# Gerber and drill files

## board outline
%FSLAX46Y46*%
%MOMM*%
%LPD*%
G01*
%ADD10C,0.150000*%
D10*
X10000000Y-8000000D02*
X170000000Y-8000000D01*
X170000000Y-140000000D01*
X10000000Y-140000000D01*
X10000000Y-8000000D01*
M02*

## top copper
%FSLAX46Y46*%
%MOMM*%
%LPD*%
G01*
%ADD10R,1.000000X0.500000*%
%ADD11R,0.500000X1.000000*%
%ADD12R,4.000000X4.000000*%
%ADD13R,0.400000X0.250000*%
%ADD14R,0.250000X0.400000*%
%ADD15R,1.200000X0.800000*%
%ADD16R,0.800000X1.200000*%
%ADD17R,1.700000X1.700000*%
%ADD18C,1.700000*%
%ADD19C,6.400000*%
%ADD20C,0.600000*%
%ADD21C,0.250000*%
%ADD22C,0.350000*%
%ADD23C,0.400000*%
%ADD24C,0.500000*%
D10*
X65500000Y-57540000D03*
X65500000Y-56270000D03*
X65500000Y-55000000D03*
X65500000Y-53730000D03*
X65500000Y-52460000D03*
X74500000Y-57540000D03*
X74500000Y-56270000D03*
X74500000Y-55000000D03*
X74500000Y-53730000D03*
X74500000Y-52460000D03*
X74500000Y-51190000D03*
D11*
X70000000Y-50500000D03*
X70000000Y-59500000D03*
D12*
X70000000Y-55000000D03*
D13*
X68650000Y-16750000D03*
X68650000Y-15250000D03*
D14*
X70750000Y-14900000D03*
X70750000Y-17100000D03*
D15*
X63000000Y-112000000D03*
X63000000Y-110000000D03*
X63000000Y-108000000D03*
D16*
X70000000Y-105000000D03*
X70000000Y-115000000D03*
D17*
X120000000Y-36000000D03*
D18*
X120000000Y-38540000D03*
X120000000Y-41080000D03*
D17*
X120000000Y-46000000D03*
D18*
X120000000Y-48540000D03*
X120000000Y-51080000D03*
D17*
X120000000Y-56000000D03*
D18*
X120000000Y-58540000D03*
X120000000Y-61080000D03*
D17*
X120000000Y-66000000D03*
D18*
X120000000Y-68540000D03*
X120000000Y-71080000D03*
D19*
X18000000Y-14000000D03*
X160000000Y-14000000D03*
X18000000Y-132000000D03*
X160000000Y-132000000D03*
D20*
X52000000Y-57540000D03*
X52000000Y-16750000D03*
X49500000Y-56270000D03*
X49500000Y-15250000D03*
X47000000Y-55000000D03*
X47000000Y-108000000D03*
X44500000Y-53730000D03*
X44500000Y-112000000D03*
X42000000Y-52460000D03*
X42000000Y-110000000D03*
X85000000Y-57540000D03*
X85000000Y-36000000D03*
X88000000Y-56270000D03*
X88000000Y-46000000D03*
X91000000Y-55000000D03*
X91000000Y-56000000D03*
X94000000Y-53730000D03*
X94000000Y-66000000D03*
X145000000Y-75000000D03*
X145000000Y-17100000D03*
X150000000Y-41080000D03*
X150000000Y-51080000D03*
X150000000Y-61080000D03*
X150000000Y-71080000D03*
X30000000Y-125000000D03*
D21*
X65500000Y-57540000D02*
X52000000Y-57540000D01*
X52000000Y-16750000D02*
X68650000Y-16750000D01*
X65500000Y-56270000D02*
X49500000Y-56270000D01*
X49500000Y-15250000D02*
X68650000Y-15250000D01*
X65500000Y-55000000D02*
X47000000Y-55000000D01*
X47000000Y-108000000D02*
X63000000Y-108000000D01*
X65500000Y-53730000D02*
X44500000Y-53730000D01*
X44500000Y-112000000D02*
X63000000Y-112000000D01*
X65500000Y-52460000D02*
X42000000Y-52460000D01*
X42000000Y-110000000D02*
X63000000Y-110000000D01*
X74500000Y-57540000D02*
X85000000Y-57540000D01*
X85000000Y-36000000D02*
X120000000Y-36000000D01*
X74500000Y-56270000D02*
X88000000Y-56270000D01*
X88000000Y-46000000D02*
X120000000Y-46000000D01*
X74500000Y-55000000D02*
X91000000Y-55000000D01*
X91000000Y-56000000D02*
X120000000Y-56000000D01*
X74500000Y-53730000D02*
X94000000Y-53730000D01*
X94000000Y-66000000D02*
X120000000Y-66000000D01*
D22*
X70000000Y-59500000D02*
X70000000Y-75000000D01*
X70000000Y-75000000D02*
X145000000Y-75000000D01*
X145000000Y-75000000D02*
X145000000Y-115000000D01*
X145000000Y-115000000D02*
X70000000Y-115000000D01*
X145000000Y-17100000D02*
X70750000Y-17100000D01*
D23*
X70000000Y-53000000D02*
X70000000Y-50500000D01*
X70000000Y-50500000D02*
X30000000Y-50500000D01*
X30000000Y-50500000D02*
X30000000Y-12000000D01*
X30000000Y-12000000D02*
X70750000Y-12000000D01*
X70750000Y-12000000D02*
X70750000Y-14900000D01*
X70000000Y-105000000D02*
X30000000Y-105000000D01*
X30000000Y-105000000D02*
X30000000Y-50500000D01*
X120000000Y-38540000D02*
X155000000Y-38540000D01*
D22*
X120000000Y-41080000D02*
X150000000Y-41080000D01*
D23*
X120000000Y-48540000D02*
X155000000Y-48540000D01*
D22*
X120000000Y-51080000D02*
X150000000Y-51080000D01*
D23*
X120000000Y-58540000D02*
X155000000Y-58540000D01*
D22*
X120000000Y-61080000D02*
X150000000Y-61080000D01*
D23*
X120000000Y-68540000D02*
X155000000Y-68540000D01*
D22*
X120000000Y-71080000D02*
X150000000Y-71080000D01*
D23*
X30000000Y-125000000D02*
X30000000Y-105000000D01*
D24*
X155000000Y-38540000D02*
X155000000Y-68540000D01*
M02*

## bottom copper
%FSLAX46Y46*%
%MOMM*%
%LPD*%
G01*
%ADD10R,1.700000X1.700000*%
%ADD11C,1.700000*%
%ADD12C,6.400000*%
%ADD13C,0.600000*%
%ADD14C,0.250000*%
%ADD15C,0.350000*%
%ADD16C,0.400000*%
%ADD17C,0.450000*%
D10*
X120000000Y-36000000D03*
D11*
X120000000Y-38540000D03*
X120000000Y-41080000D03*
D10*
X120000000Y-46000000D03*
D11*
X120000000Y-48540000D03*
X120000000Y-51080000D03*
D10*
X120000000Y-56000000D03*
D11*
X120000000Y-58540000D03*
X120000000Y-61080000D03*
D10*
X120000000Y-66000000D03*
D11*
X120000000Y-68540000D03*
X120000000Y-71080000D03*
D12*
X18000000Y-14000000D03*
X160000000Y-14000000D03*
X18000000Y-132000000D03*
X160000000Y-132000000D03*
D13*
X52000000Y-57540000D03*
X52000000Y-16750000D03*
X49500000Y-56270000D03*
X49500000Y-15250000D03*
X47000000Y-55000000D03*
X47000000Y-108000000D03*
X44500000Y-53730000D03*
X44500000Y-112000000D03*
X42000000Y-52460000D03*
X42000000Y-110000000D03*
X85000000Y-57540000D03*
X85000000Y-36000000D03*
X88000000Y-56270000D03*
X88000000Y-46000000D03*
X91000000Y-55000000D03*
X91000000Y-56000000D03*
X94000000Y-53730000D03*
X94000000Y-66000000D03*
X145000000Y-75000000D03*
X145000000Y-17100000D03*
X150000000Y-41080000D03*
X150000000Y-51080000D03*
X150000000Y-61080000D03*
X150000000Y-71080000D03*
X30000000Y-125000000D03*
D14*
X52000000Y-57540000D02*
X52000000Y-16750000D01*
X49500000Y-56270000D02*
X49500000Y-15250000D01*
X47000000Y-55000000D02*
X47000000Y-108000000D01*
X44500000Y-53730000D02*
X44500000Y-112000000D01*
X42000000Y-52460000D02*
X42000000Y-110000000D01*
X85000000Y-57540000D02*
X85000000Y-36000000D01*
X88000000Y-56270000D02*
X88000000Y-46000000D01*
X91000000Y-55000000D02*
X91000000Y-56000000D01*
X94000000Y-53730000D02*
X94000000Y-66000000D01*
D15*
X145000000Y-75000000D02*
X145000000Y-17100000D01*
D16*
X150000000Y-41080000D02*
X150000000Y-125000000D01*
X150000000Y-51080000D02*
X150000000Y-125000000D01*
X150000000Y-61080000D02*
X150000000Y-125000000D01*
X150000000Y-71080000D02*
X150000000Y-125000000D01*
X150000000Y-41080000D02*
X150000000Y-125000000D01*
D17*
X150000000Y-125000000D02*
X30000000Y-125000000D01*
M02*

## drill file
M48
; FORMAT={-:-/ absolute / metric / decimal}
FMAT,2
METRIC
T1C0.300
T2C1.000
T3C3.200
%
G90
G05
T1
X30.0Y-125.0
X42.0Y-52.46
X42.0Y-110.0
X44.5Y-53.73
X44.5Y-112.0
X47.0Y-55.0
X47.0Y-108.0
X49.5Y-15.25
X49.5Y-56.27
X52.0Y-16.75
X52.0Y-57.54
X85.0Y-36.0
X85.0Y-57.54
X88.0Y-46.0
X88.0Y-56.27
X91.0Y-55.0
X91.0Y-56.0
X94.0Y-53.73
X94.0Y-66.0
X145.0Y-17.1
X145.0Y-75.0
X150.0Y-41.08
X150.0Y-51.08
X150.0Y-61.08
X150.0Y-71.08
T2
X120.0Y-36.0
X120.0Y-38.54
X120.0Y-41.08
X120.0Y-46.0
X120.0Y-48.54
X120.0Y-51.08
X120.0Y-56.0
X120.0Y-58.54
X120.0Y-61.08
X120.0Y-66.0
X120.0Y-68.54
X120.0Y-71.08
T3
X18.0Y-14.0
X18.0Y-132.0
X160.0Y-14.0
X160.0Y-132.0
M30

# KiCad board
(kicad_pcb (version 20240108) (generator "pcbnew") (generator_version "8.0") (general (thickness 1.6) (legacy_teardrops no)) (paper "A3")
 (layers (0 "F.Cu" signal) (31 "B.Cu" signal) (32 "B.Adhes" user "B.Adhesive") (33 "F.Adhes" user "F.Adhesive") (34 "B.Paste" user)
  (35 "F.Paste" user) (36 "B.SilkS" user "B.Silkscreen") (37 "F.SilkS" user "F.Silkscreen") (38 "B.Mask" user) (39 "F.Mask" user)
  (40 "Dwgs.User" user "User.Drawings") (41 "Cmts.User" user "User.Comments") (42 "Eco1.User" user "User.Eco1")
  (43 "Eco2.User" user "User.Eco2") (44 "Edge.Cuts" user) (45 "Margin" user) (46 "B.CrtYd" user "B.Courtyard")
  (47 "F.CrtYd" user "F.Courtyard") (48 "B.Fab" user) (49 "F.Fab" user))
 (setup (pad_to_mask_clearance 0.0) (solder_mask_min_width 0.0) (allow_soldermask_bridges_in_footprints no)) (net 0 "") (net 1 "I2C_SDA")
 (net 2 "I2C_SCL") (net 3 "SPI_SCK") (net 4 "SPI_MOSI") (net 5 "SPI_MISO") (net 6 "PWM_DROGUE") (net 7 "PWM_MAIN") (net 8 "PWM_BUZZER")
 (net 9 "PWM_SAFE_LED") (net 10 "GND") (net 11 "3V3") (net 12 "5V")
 (gr_rect (start 10 8) (end 170 140) (stroke (width 0.15) (type solid)) (fill none) (layer "Edge.Cuts"))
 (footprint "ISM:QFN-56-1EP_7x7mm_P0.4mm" (layer "F.Cu") (at 70 55)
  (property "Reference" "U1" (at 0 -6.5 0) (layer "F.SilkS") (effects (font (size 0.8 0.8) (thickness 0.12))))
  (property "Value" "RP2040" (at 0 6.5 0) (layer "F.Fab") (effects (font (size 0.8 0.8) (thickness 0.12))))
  (pad "1" smd rect (at -4.5 2.54) (size 1.0 0.5) (layers "F.Cu" "F.Paste" "F.Mask") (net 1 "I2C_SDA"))
  (pad "2" smd rect (at -4.5 1.27) (size 1.0 0.5) (layers "F.Cu" "F.Paste" "F.Mask") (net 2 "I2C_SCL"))
  (pad "3" smd rect (at -4.5 0) (size 1.0 0.5) (layers "F.Cu" "F.Paste" "F.Mask") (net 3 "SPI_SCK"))
  (pad "4" smd rect (at -4.5 -1.27) (size 1.0 0.5) (layers "F.Cu" "F.Paste" "F.Mask") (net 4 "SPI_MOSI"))
  (pad "5" smd rect (at -4.5 -2.54) (size 1.0 0.5) (layers "F.Cu" "F.Paste" "F.Mask") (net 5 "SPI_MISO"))
  (pad "6" smd rect (at 4.5 2.54) (size 1.0 0.5) (layers "F.Cu" "F.Paste" "F.Mask") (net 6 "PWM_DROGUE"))
  (pad "7" smd rect (at 4.5 1.27) (size 1.0 0.5) (layers "F.Cu" "F.Paste" "F.Mask") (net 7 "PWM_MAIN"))
  (pad "8" smd rect (at 4.5 0) (size 1.0 0.5) (layers "F.Cu" "F.Paste" "F.Mask") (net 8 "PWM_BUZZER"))
  (pad "9" smd rect (at 4.5 -1.27) (size 1.0 0.5) (layers "F.Cu" "F.Paste" "F.Mask") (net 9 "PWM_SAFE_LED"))
  (pad "12" smd rect (at 4.5 -2.54) (size 1.0 0.5) (layers "F.Cu" "F.Paste" "F.Mask"))
  (pad "13" smd rect (at 4.5 -3.81) (size 1.0 0.5) (layers "F.Cu" "F.Paste" "F.Mask"))
  (pad "10" smd rect (at 0 -4.5) (size 0.5 1.0) (layers "F.Cu" "F.Paste" "F.Mask") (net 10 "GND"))
  (pad "11" smd rect (at 0 4.5) (size 0.5 1.0) (layers "F.Cu" "F.Paste" "F.Mask") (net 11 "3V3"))
  (pad "EP" smd rect (at 0 0) (size 4 4) (layers "F.Cu" "F.Paste" "F.Mask") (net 10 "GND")))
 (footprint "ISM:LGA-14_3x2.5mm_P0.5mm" (layer "F.Cu") (at 70 16)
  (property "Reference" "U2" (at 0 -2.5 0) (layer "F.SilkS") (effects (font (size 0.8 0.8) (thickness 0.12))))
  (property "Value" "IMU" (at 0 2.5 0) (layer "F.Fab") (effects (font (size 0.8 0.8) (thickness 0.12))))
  (pad "1" smd rect (at -1.35 0.75) (size 0.4 0.25) (layers "F.Cu" "F.Paste" "F.Mask") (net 1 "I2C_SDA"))
  (pad "2" smd rect (at -1.35 -0.75) (size 0.4 0.25) (layers "F.Cu" "F.Paste" "F.Mask") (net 2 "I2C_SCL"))
  (pad "3" smd rect (at 0.75 -1.1) (size 0.25 0.4) (layers "F.Cu" "F.Paste" "F.Mask") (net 10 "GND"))
  (pad "4" smd rect (at 0.75 1.1) (size 0.25 0.4) (layers "F.Cu" "F.Paste" "F.Mask") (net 11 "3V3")))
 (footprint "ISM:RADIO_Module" (layer "F.Cu") (at 70 110)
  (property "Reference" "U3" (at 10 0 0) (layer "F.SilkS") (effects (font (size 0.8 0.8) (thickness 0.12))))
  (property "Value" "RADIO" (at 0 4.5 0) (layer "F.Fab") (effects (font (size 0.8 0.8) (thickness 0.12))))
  (pad "1" smd rect (at -7 2) (size 1.2 0.8) (layers "F.Cu" "F.Paste" "F.Mask") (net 4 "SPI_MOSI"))
  (pad "2" smd rect (at -7 0) (size 1.2 0.8) (layers "F.Cu" "F.Paste" "F.Mask") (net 5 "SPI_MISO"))
  (pad "3" smd rect (at -7 -2) (size 1.2 0.8) (layers "F.Cu" "F.Paste" "F.Mask") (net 3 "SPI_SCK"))
  (pad "4" smd rect (at 0 -5) (size 0.8 1.2) (layers "F.Cu" "F.Paste" "F.Mask") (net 10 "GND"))
  (pad "5" smd rect (at 0 5) (size 0.8 1.2) (layers "F.Cu" "F.Paste" "F.Mask") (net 11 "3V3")))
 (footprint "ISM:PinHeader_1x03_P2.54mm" (layer "F.Cu") (at 120 36)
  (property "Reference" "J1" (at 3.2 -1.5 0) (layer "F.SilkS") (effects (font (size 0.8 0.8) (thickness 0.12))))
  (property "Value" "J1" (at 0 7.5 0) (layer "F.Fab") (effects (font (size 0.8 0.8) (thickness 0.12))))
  (pad "1" thru_hole rect (at 0 0) (size 1.7 1.7) (drill 1.0) (layers "*.Cu" "*.Mask") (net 6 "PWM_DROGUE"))
  (pad "2" thru_hole circle (at 0 2.54) (size 1.7 1.7) (drill 1.0) (layers "*.Cu" "*.Mask") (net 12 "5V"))
  (pad "3" thru_hole circle (at 0 5.08) (size 1.7 1.7) (drill 1.0) (layers "*.Cu" "*.Mask") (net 10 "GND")))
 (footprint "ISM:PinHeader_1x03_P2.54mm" (layer "F.Cu") (at 120 46)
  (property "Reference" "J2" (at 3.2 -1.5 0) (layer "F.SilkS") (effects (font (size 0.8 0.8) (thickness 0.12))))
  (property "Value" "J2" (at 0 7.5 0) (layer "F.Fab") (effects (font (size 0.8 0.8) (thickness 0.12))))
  (pad "1" thru_hole rect (at 0 0) (size 1.7 1.7) (drill 1.0) (layers "*.Cu" "*.Mask") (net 7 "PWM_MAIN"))
  (pad "2" thru_hole circle (at 0 2.54) (size 1.7 1.7) (drill 1.0) (layers "*.Cu" "*.Mask") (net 12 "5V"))
  (pad "3" thru_hole circle (at 0 5.08) (size 1.7 1.7) (drill 1.0) (layers "*.Cu" "*.Mask") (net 10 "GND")))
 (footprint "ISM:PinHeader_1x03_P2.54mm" (layer "F.Cu") (at 120 56)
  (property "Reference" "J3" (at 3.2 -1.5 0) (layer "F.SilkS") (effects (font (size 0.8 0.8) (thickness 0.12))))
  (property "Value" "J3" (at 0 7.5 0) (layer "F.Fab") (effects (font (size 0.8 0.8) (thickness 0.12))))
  (pad "1" thru_hole rect (at 0 0) (size 1.7 1.7) (drill 1.0) (layers "*.Cu" "*.Mask") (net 8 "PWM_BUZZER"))
  (pad "2" thru_hole circle (at 0 2.54) (size 1.7 1.7) (drill 1.0) (layers "*.Cu" "*.Mask") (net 12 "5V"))
  (pad "3" thru_hole circle (at 0 5.08) (size 1.7 1.7) (drill 1.0) (layers "*.Cu" "*.Mask") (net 10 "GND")))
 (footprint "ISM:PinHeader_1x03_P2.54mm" (layer "F.Cu") (at 120 66)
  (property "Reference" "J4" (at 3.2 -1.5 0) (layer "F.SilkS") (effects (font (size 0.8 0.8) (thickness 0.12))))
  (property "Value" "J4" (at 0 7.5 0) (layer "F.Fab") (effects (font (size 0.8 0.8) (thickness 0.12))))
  (pad "1" thru_hole rect (at 0 0) (size 1.7 1.7) (drill 1.0) (layers "*.Cu" "*.Mask") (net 9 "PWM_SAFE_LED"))
  (pad "2" thru_hole circle (at 0 2.54) (size 1.7 1.7) (drill 1.0) (layers "*.Cu" "*.Mask") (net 12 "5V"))
  (pad "3" thru_hole circle (at 0 5.08) (size 1.7 1.7) (drill 1.0) (layers "*.Cu" "*.Mask") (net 10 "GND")))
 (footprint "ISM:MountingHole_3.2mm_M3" (layer "F.Cu") (at 18 14)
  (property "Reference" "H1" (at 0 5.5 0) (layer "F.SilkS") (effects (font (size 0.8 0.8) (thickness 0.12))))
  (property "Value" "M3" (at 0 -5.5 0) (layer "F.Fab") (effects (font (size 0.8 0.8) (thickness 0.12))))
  (pad "" thru_hole circle (at 0 0) (size 6.4 6.4) (drill 3.2) (layers "*.Cu" "*.Mask")))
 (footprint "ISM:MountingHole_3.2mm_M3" (layer "F.Cu") (at 160 14)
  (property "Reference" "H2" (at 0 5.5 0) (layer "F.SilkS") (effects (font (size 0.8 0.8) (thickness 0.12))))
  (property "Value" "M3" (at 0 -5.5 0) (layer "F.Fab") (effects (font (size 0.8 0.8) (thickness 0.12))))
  (pad "" thru_hole circle (at 0 0) (size 6.4 6.4) (drill 3.2) (layers "*.Cu" "*.Mask")))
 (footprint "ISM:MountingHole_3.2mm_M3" (layer "F.Cu") (at 18 132)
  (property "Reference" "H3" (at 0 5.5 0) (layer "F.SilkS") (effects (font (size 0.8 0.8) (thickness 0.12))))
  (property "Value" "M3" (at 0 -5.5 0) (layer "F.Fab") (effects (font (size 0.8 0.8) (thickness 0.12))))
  (pad "" thru_hole circle (at 0 0) (size 6.4 6.4) (drill 3.2) (layers "*.Cu" "*.Mask")))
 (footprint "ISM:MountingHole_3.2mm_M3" (layer "F.Cu") (at 160 132)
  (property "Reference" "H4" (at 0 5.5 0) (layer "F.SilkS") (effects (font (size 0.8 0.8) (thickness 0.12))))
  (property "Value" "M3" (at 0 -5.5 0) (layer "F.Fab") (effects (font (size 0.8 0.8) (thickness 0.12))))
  (pad "" thru_hole circle (at 0 0) (size 6.4 6.4) (drill 3.2) (layers "*.Cu" "*.Mask")))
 (segment (start 65.5 57.54) (end 52.0 57.54) (width 0.25) (layer "F.Cu") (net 1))
 (segment (start 52.0 57.54) (end 52.0 16.75) (width 0.25) (layer "B.Cu") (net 1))
 (segment (start 52.0 16.75) (end 68.65 16.75) (width 0.25) (layer "F.Cu") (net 1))
 (segment (start 65.5 56.27) (end 49.5 56.27) (width 0.25) (layer "F.Cu") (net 2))
 (segment (start 49.5 56.27) (end 49.5 15.25) (width 0.25) (layer "B.Cu") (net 2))
 (segment (start 49.5 15.25) (end 68.65 15.25) (width 0.25) (layer "F.Cu") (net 2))
 (segment (start 65.5 55) (end 47.0 55) (width 0.25) (layer "F.Cu") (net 3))
 (segment (start 47.0 55) (end 47.0 108) (width 0.25) (layer "B.Cu") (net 3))
 (segment (start 47.0 108) (end 63 108) (width 0.25) (layer "F.Cu") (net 3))
 (segment (start 65.5 53.73) (end 44.5 53.73) (width 0.25) (layer "F.Cu") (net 4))
 (segment (start 44.5 53.73) (end 44.5 112) (width 0.25) (layer "B.Cu") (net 4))
 (segment (start 44.5 112) (end 63 112) (width 0.25) (layer "F.Cu") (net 4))
 (segment (start 65.5 52.46) (end 42.0 52.46) (width 0.25) (layer "F.Cu") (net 5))
 (segment (start 42.0 52.46) (end 42.0 110) (width 0.25) (layer "B.Cu") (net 5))
 (segment (start 42.0 110) (end 63 110) (width 0.25) (layer "F.Cu") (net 5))
 (segment (start 74.5 57.54) (end 85 57.54) (width 0.25) (layer "F.Cu") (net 6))
 (segment (start 85 57.54) (end 85 36) (width 0.25) (layer "B.Cu") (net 6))
 (segment (start 85 36) (end 120 36) (width 0.25) (layer "F.Cu") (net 6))
 (segment (start 74.5 56.27) (end 88 56.27) (width 0.25) (layer "F.Cu") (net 7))
 (segment (start 88 56.27) (end 88 46) (width 0.25) (layer "B.Cu") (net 7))
 (segment (start 88 46) (end 120 46) (width 0.25) (layer "F.Cu") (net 7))
 (segment (start 74.5 55) (end 91 55) (width 0.25) (layer "F.Cu") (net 8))
 (segment (start 91 55) (end 91 56) (width 0.25) (layer "B.Cu") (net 8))
 (segment (start 91 56) (end 120 56) (width 0.25) (layer "F.Cu") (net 8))
 (segment (start 74.5 53.73) (end 94 53.73) (width 0.25) (layer "F.Cu") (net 9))
 (segment (start 94 53.73) (end 94 66) (width 0.25) (layer "B.Cu") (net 9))
 (segment (start 94 66) (end 120 66) (width 0.25) (layer "F.Cu") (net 9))
 (segment (start 70 59.5) (end 70 75) (width 0.35) (layer "F.Cu") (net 11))
 (segment (start 70 75) (end 145 75) (width 0.35) (layer "F.Cu") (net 11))
 (segment (start 145 75) (end 145 115) (width 0.35) (layer "F.Cu") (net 11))
 (segment (start 145 115) (end 70 115) (width 0.35) (layer "F.Cu") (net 11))
 (segment (start 145 75) (end 145 17.1) (width 0.35) (layer "B.Cu") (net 11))
 (segment (start 145 17.1) (end 70.75 17.1) (width 0.35) (layer "F.Cu") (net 11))
 (segment (start 70 53) (end 70 50.5) (width 0.4) (layer "F.Cu") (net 10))
 (segment (start 70 50.5) (end 30 50.5) (width 0.4) (layer "F.Cu") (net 10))
 (segment (start 30 50.5) (end 30 12) (width 0.4) (layer "F.Cu") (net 10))
 (segment (start 30 12) (end 70.75 12) (width 0.4) (layer "F.Cu") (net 10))
 (segment (start 70.75 12) (end 70.75 14.9) (width 0.4) (layer "F.Cu") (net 10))
 (segment (start 70 105) (end 30 105) (width 0.4) (layer "F.Cu") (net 10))
 (segment (start 30 105) (end 30 50.5) (width 0.4) (layer "F.Cu") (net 10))
 (segment (start 120 38.54) (end 155 38.54) (width 0.4) (layer "F.Cu") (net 12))
 (segment (start 120 41.08) (end 150 41.08) (width 0.35) (layer "F.Cu") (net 10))
 (segment (start 150 41.08) (end 150 125) (width 0.4) (layer "B.Cu") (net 10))
 (segment (start 120 48.54) (end 155 48.54) (width 0.4) (layer "F.Cu") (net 12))
 (segment (start 120 51.08) (end 150 51.08) (width 0.35) (layer "F.Cu") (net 10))
 (segment (start 150 51.08) (end 150 125) (width 0.4) (layer "B.Cu") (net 10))
 (segment (start 120 58.54) (end 155 58.54) (width 0.4) (layer "F.Cu") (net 12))
 (segment (start 120 61.08) (end 150 61.08) (width 0.35) (layer "F.Cu") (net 10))
 (segment (start 150 61.08) (end 150 125) (width 0.4) (layer "B.Cu") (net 10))
 (segment (start 120 68.54) (end 155 68.54) (width 0.4) (layer "F.Cu") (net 12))
 (segment (start 120 71.08) (end 150 71.08) (width 0.35) (layer "F.Cu") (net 10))
 (segment (start 150 71.08) (end 150 125) (width 0.4) (layer "B.Cu") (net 10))
 (segment (start 150 41.08) (end 150 125) (width 0.4) (layer "B.Cu") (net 10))
 (segment (start 150 125) (end 30 125) (width 0.45) (layer "B.Cu") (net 10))
 (segment (start 30 125) (end 30 105) (width 0.4) (layer "F.Cu") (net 10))
 (segment (start 155 38.54) (end 155 68.54) (width 0.5) (layer "F.Cu") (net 12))
 (via (at 52.0 57.54) (size 0.6) (drill 0.3) (layers "F.Cu" "B.Cu") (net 1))
 (via (at 52.0 16.75) (size 0.6) (drill 0.3) (layers "F.Cu" "B.Cu") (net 1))
 (via (at 49.5 56.27) (size 0.6) (drill 0.3) (layers "F.Cu" "B.Cu") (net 2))
 (via (at 49.5 15.25) (size 0.6) (drill 0.3) (layers "F.Cu" "B.Cu") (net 2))
 (via (at 47.0 55) (size 0.6) (drill 0.3) (layers "F.Cu" "B.Cu") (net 3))
 (via (at 47.0 108) (size 0.6) (drill 0.3) (layers "F.Cu" "B.Cu") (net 3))
 (via (at 44.5 53.73) (size 0.6) (drill 0.3) (layers "F.Cu" "B.Cu") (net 4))
 (via (at 44.5 112) (size 0.6) (drill 0.3) (layers "F.Cu" "B.Cu") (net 4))
 (via (at 42.0 52.46) (size 0.6) (drill 0.3) (layers "F.Cu" "B.Cu") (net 5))
 (via (at 42.0 110) (size 0.6) (drill 0.3) (layers "F.Cu" "B.Cu") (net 5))
 (via (at 85 57.54) (size 0.6) (drill 0.3) (layers "F.Cu" "B.Cu") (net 6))
 (via (at 85 36) (size 0.6) (drill 0.3) (layers "F.Cu" "B.Cu") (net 6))
 (via (at 88 56.27) (size 0.6) (drill 0.3) (layers "F.Cu" "B.Cu") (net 7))
 (via (at 88 46) (size 0.6) (drill 0.3) (layers "F.Cu" "B.Cu") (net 7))
 (via (at 91 55) (size 0.6) (drill 0.3) (layers "F.Cu" "B.Cu") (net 8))
 (via (at 91 56) (size 0.6) (drill 0.3) (layers "F.Cu" "B.Cu") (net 8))
 (via (at 94 53.73) (size 0.6) (drill 0.3) (layers "F.Cu" "B.Cu") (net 9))
 (via (at 94 66) (size 0.6) (drill 0.3) (layers "F.Cu" "B.Cu") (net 9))
 (via (at 145 75) (size 0.6) (drill 0.3) (layers "F.Cu" "B.Cu") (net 11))
 (via (at 145 17.1) (size 0.6) (drill 0.3) (layers "F.Cu" "B.Cu") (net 11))
 (via (at 150 41.08) (size 0.6) (drill 0.3) (layers "F.Cu" "B.Cu") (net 10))
 (via (at 150 51.08) (size 0.6) (drill 0.3) (layers "F.Cu" "B.Cu") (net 10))
 (via (at 150 61.08) (size 0.6) (drill 0.3) (layers "F.Cu" "B.Cu") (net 10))
 (via (at 150 71.08) (size 0.6) (drill 0.3) (layers "F.Cu" "B.Cu") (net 10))
 (via (at 30 125) (size 0.6) (drill 0.3) (layers "F.Cu" "B.Cu") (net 10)))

